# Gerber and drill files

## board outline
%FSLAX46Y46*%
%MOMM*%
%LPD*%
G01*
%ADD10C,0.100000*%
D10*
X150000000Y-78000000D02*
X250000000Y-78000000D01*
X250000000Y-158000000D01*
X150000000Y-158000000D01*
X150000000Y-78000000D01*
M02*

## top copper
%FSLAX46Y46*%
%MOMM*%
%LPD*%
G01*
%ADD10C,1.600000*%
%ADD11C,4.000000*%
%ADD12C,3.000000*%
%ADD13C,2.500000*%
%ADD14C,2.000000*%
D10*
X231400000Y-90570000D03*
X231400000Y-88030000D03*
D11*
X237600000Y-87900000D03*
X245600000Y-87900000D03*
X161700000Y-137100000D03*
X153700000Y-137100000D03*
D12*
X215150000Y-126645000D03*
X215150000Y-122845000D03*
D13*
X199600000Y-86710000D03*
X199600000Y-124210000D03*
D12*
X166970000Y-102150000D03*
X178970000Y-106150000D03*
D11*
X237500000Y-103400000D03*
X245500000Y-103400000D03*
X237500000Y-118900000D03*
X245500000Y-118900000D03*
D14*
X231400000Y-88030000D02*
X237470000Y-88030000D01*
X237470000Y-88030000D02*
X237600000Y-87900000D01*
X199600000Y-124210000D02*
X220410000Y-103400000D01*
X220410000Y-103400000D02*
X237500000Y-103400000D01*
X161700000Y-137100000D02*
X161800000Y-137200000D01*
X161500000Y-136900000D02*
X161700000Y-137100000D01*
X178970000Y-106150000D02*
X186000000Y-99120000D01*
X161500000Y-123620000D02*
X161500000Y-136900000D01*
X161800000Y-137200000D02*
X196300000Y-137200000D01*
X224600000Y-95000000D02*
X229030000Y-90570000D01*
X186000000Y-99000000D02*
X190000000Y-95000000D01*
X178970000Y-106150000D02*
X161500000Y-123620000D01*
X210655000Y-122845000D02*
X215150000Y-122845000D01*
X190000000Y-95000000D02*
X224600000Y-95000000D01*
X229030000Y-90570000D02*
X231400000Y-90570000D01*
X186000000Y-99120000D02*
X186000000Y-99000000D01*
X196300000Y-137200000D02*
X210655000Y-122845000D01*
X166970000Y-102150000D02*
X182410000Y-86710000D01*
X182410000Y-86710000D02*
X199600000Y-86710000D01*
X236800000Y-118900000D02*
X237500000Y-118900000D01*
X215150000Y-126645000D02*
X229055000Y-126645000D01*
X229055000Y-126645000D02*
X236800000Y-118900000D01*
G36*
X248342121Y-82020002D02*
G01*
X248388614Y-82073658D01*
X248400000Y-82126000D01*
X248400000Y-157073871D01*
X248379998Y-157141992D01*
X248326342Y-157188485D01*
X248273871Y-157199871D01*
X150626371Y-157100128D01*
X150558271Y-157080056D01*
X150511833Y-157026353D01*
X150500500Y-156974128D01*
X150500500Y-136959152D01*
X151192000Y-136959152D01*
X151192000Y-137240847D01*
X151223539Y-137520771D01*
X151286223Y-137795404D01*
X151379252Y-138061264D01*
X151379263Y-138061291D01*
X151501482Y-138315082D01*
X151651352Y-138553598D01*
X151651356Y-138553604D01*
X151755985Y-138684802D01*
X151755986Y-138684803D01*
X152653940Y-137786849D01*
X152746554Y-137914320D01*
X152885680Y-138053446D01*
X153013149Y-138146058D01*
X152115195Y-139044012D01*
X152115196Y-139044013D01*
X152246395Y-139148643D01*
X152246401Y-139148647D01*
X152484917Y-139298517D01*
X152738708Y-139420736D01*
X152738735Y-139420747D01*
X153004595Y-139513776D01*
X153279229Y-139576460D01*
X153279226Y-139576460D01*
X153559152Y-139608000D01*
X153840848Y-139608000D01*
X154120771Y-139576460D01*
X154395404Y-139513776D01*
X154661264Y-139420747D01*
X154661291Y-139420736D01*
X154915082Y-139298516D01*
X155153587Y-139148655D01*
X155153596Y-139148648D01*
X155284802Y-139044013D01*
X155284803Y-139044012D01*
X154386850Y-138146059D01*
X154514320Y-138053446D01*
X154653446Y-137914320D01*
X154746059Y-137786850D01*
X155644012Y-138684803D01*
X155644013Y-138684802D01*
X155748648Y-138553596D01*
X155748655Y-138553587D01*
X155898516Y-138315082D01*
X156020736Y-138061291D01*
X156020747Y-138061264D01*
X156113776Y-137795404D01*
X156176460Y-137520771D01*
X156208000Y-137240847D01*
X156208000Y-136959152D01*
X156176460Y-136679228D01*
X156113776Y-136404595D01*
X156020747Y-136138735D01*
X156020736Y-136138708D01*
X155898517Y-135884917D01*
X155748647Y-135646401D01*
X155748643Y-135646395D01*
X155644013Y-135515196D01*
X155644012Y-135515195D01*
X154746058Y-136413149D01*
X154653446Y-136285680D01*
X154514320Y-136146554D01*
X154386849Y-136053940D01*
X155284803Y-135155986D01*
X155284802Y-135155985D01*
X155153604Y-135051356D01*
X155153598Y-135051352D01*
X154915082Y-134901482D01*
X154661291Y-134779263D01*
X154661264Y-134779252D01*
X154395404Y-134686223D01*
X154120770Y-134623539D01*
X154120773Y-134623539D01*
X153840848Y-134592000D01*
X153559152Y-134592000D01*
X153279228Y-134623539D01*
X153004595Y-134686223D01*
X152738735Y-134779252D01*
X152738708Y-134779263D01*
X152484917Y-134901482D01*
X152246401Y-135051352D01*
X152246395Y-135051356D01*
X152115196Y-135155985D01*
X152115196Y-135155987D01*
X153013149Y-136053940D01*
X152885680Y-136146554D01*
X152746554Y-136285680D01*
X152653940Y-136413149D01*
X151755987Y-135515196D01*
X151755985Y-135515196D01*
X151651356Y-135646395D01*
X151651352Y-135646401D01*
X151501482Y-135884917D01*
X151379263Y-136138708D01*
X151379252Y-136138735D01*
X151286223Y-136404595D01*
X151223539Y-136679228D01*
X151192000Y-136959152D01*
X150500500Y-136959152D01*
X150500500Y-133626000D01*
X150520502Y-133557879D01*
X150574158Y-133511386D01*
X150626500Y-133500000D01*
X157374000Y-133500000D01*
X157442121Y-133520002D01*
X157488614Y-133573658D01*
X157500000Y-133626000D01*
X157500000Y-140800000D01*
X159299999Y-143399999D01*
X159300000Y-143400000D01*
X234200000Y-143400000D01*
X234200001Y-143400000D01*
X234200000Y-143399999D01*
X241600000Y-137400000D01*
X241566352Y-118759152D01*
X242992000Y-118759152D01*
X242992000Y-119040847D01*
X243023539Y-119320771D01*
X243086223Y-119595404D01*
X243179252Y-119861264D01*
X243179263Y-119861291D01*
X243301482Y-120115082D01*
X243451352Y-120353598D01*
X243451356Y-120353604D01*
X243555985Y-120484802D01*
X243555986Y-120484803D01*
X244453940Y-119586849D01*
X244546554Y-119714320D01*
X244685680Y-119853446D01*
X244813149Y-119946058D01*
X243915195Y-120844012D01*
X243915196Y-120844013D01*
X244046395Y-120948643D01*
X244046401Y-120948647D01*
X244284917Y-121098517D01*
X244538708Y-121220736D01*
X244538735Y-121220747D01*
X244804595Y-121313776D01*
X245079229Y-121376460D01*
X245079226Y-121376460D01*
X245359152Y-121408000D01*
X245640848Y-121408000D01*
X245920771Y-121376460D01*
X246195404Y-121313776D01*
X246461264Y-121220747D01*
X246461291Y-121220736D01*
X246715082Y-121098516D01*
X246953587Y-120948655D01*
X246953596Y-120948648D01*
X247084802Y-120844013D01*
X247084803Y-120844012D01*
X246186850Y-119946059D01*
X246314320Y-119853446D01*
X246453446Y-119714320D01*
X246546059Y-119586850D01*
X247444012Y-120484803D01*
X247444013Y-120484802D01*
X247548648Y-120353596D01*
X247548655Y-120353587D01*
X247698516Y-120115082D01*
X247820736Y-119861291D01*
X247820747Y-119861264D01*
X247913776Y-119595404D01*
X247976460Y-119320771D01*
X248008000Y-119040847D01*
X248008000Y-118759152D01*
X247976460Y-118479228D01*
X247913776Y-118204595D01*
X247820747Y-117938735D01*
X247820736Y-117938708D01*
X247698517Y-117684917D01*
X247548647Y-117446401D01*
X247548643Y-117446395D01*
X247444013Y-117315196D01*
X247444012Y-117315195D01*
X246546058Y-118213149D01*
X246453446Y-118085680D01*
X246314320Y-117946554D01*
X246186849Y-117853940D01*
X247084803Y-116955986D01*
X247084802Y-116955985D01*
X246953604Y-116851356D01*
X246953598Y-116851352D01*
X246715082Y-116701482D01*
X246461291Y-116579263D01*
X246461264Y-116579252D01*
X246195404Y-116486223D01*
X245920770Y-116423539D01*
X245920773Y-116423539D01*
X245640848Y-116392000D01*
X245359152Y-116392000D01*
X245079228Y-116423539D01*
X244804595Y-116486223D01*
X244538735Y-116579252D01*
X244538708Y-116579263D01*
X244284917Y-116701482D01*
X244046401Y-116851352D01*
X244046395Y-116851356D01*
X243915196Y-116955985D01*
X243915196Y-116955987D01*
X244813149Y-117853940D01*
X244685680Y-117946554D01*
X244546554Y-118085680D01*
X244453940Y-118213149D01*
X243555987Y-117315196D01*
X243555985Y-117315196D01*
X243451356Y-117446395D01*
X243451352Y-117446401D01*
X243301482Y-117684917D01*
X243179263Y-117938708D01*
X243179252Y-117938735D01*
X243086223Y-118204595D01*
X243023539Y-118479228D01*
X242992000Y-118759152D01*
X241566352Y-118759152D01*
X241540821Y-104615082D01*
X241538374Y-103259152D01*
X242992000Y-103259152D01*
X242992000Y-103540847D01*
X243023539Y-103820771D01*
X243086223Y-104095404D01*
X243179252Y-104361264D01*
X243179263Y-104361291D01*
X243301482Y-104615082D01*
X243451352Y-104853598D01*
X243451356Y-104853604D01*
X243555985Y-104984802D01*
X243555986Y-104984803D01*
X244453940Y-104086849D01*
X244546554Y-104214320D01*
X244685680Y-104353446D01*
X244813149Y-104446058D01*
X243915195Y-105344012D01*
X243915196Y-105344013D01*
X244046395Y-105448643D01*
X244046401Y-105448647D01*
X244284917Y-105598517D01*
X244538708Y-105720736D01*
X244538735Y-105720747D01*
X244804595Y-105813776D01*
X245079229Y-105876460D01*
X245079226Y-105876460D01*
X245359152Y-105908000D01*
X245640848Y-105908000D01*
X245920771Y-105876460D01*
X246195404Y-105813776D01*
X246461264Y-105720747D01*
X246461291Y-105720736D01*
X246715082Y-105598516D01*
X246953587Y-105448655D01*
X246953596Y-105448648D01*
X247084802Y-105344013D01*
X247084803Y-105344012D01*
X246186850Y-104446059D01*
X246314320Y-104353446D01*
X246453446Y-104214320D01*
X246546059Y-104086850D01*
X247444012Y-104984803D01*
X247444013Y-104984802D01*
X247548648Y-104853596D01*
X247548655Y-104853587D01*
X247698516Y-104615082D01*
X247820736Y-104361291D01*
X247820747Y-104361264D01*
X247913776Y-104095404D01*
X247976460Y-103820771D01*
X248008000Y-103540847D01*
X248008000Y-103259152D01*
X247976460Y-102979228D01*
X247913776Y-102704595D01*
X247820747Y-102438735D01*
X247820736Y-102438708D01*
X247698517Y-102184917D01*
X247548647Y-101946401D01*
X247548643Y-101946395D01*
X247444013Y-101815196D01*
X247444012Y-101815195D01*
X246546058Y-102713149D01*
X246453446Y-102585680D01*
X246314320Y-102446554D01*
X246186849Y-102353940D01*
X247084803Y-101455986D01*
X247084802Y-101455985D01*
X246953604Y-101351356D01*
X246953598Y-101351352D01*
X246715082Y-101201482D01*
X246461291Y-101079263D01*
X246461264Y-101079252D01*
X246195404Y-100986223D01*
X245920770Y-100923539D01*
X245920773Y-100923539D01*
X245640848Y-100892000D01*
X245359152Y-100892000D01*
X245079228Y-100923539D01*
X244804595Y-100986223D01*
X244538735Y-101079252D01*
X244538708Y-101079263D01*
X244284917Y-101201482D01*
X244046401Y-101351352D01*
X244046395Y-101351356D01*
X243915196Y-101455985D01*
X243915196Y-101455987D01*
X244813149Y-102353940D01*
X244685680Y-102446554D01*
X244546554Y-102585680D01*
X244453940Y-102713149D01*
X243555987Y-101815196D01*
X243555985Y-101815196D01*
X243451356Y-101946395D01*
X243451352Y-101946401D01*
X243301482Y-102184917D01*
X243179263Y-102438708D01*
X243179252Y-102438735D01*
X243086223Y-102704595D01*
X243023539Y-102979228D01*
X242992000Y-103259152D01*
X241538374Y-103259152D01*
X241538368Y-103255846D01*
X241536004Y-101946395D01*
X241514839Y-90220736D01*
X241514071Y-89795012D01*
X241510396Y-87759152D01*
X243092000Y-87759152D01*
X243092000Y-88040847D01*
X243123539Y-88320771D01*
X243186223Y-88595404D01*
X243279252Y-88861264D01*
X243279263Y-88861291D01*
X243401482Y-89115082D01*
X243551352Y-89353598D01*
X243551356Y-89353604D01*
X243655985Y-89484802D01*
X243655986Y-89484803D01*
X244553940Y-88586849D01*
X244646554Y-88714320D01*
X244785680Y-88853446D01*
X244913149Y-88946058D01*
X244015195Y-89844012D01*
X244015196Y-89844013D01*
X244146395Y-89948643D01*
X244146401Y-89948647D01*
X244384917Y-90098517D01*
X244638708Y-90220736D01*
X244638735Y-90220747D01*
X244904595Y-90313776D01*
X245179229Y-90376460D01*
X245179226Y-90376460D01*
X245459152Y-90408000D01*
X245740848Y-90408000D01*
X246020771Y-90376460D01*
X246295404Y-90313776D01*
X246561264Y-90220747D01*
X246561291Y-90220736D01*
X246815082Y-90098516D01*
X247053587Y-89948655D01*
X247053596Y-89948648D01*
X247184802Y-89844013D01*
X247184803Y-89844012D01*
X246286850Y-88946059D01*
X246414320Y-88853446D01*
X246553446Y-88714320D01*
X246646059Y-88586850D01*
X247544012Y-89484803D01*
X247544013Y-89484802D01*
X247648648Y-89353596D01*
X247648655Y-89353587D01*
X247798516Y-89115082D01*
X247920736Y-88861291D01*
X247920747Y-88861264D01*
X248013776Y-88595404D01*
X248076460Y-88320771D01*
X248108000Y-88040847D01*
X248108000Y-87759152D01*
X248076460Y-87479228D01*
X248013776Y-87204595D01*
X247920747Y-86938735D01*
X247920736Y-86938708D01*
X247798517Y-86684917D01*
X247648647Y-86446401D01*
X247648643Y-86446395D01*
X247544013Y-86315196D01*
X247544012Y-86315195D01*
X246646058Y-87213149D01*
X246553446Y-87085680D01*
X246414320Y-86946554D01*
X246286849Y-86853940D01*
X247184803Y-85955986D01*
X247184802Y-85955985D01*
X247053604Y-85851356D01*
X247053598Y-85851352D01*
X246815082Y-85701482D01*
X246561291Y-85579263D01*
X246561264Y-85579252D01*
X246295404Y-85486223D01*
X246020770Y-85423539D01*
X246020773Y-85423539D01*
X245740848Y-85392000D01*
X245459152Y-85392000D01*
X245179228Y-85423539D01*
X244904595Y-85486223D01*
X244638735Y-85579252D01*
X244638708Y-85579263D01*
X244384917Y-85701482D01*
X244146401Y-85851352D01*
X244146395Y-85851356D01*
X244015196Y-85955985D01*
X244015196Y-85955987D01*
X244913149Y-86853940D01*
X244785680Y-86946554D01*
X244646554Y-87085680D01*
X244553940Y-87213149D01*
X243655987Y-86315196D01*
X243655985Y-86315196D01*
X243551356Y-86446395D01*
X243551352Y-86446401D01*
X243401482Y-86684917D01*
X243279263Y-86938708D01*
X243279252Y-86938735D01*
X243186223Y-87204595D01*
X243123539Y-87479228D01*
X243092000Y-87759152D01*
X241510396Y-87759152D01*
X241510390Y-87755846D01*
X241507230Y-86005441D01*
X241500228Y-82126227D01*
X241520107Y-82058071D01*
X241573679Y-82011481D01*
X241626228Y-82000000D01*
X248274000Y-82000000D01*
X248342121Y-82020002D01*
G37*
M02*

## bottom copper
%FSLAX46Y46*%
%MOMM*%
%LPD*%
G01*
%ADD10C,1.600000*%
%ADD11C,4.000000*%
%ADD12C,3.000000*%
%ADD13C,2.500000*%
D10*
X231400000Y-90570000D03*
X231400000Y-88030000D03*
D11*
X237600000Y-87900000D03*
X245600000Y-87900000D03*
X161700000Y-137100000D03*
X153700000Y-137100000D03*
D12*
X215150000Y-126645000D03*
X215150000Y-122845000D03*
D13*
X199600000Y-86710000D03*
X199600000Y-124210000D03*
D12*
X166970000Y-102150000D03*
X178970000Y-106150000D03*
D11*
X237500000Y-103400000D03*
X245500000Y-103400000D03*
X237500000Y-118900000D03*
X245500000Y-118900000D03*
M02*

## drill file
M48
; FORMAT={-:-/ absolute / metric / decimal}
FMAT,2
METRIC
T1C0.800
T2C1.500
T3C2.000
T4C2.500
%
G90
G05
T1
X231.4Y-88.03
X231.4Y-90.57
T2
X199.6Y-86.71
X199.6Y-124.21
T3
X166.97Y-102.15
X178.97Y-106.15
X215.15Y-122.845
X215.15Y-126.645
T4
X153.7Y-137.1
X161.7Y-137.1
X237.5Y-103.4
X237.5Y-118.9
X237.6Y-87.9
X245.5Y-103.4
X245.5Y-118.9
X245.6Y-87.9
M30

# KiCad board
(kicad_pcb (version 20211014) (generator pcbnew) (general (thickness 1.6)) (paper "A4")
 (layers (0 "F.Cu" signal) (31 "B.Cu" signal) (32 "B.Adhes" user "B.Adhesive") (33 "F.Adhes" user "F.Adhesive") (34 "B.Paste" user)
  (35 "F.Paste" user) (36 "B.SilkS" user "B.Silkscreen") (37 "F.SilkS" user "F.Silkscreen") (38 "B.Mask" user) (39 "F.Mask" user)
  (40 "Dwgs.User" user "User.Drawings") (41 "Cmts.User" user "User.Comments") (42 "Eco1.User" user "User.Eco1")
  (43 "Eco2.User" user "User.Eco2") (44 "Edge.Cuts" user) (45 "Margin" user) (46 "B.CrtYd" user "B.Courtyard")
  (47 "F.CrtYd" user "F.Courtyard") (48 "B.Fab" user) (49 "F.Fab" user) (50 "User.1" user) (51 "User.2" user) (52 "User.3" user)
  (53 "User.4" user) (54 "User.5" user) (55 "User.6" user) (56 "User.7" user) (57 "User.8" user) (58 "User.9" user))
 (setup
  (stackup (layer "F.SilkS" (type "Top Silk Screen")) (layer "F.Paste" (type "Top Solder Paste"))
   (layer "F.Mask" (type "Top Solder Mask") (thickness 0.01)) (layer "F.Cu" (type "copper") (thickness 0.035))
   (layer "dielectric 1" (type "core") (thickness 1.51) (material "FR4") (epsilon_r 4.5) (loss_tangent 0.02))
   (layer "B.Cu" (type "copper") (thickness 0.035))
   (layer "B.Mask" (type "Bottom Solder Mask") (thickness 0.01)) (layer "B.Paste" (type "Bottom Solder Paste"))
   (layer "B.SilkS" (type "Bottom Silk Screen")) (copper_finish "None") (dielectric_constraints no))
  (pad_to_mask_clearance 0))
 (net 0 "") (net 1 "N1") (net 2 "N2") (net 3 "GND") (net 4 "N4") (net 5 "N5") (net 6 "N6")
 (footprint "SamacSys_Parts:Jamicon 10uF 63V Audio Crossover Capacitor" (layer "F.Cu") (at 231.4 90.63 180)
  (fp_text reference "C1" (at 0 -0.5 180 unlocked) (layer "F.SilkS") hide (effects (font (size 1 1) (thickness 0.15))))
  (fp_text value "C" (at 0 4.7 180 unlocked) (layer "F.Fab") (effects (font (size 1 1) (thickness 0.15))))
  (pad "1" thru_hole circle (at 0 0.06 180) (size 1.6 1.6) (drill 0.8) (layers *.Cu *.Mask) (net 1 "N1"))
  (pad "2" thru_hole circle (at 0 2.6 180) (size 1.6 1.6) (drill 0.8) (layers *.Cu *.Mask) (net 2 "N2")))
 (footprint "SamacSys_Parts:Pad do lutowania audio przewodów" (layer "F.Cu") (at 244.1 87.9)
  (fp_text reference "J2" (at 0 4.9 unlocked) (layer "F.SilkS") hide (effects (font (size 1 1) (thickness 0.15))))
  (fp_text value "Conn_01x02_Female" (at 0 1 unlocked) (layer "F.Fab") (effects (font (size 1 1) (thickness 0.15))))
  (pad "1" thru_hole circle (at -6.5 0) (size 4 4) (drill 2.5) (layers *.Cu *.Mask) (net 2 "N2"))
  (pad "2" thru_hole circle (at 1.5 0) (size 4 4) (drill 2.5) (layers *.Cu *.Mask) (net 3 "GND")))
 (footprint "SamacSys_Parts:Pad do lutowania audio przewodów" (layer "F.Cu") (at 155.2 137.1 180)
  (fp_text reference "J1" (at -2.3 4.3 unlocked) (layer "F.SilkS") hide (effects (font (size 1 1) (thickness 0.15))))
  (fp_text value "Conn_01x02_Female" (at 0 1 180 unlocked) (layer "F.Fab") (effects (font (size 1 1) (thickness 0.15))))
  (pad "1" thru_hole circle (at -6.5 0 180) (size 4 4) (drill 2.5) (layers *.Cu *.Mask) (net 1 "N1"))
  (pad "2" thru_hole circle (at 1.5 0 180) (size 4 4) (drill 2.5) (layers *.Cu *.Mask) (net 3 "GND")))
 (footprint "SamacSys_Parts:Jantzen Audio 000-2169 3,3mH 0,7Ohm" (layer "F.Cu") (at 214.8 136.795 -90)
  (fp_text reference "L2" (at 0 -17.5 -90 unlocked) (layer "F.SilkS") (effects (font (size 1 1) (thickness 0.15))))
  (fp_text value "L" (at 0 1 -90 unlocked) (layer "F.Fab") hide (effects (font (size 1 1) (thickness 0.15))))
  (pad "1" thru_hole circle (at -10.15 -0.35 270) (size 3 3) (drill 2) (layers *.Cu *.Mask) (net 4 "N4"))
  (pad "2" thru_hole circle (at -13.95 -0.35 270) (size 3 3) (drill 2) (layers *.Cu *.Mask) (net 1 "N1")))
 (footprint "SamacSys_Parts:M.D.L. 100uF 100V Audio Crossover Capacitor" (layer "F.Cu") (at 199.6 86.91 -90)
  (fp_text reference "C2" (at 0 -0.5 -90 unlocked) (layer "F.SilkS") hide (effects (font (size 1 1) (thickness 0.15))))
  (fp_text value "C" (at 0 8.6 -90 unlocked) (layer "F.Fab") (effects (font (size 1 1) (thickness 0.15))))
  (pad "1" thru_hole circle (at -0.2 0 270) (size 2.5 2.5) (drill 1.5) (layers *.Cu *.Mask) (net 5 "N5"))
  (pad "2" thru_hole circle (at 37.3 0 270) (size 2.5 2.5) (drill 1.5) (layers *.Cu *.Mask) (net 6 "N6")))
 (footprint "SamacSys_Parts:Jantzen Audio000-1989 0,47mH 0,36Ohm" (layer "F.Cu") (at 166.97 97.15)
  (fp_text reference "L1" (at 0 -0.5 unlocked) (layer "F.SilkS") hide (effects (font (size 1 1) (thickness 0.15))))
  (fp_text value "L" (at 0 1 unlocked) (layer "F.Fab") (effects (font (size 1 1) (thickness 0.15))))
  (pad "1" thru_hole circle (at 0 5) (size 3 3) (drill 2) (layers *.Cu *.Mask) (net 5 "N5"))
  (pad "2" thru_hole circle (at 12 9) (size 3 3) (drill 2) (layers *.Cu *.Mask) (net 1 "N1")))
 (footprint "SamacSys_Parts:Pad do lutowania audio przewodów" (layer "F.Cu") (at 244 103.4)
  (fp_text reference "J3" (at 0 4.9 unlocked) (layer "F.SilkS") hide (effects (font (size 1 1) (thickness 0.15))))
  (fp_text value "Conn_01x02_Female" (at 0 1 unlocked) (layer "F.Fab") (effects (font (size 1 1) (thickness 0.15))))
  (pad "1" thru_hole circle (at -6.5 0) (size 4 4) (drill 2.5) (layers *.Cu *.Mask) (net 6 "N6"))
  (pad "2" thru_hole circle (at 1.5 0) (size 4 4) (drill 2.5) (layers *.Cu *.Mask) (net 3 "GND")))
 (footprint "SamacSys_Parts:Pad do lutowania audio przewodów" (layer "F.Cu") (at 244 118.9)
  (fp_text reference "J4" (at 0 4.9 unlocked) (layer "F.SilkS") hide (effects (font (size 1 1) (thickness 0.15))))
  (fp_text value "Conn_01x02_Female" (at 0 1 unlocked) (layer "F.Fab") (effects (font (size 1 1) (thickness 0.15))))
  (pad "1" thru_hole circle (at -6.5 0) (size 4 4) (drill 2.5) (layers *.Cu *.Mask) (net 4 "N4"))
  (pad "2" thru_hole circle (at 1.5 0) (size 4 4) (drill 2.5) (layers *.Cu *.Mask) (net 3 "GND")))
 (gr_rect (start 150 78) (end 250 158) (layer "Edge.Cuts") (width 0.1) (fill none))
 (segment (start 231.4 88.03) (end 237.47 88.03) (width 2) (layer "F.Cu") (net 2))
 (segment (start 237.47 88.03) (end 237.6 87.9) (width 2) (layer "F.Cu") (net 2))
 (segment (start 199.6 124.21) (end 220.41 103.4) (width 2) (layer "F.Cu") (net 6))
 (segment (start 220.41 103.4) (end 237.5 103.4) (width 2) (layer "F.Cu") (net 6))
 (segment (start 161.7 137.1) (end 161.8 137.2) (width 2) (layer "F.Cu") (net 1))
 (segment (start 161.5 136.9) (end 161.7 137.1) (width 2) (layer "F.Cu") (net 1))
 (segment (start 178.97 106.15) (end 186 99.12) (width 2) (layer "F.Cu") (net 1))
 (segment (start 161.5 123.62) (end 161.5 136.9) (width 2) (layer "F.Cu") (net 1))
 (segment (start 161.8 137.2) (end 196.3 137.2) (width 2) (layer "F.Cu") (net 1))
 (segment (start 224.6 95) (end 229.03 90.57) (width 2) (layer "F.Cu") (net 1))
 (segment (start 186 99) (end 190 95) (width 2) (layer "F.Cu") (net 1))
 (segment (start 178.97 106.15) (end 161.5 123.62) (width 2) (layer "F.Cu") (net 1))
 (segment (start 210.655 122.845) (end 215.15 122.845) (width 2) (layer "F.Cu") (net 1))
 (segment (start 190 95) (end 224.6 95) (width 2) (layer "F.Cu") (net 1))
 (segment (start 229.03 90.57) (end 231.4 90.57) (width 2) (layer "F.Cu") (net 1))
 (segment (start 186 99.12) (end 186 99) (width 2) (layer "F.Cu") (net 1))
 (segment (start 196.3 137.2) (end 210.655 122.845) (width 2) (layer "F.Cu") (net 1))
 (segment (start 166.97 102.15) (end 182.41 86.71) (width 2) (layer "F.Cu") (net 5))
 (segment (start 182.41 86.71) (end 199.6 86.71) (width 2) (layer "F.Cu") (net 5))
 (segment (start 236.8 118.9) (end 237.5 118.9) (width 2) (layer "F.Cu") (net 4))
 (segment (start 215.15 126.645) (end 229.055 126.645) (width 2) (layer "F.Cu") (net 4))
 (segment (start 229.055 126.645) (end 236.8 118.9) (width 2) (layer "F.Cu") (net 4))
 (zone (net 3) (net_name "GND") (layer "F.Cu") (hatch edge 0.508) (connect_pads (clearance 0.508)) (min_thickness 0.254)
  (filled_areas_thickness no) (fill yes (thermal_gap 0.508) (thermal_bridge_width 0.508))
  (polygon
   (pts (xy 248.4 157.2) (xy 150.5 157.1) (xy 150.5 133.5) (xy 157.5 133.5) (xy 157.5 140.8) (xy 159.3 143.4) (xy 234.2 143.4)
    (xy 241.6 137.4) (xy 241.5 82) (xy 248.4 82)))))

